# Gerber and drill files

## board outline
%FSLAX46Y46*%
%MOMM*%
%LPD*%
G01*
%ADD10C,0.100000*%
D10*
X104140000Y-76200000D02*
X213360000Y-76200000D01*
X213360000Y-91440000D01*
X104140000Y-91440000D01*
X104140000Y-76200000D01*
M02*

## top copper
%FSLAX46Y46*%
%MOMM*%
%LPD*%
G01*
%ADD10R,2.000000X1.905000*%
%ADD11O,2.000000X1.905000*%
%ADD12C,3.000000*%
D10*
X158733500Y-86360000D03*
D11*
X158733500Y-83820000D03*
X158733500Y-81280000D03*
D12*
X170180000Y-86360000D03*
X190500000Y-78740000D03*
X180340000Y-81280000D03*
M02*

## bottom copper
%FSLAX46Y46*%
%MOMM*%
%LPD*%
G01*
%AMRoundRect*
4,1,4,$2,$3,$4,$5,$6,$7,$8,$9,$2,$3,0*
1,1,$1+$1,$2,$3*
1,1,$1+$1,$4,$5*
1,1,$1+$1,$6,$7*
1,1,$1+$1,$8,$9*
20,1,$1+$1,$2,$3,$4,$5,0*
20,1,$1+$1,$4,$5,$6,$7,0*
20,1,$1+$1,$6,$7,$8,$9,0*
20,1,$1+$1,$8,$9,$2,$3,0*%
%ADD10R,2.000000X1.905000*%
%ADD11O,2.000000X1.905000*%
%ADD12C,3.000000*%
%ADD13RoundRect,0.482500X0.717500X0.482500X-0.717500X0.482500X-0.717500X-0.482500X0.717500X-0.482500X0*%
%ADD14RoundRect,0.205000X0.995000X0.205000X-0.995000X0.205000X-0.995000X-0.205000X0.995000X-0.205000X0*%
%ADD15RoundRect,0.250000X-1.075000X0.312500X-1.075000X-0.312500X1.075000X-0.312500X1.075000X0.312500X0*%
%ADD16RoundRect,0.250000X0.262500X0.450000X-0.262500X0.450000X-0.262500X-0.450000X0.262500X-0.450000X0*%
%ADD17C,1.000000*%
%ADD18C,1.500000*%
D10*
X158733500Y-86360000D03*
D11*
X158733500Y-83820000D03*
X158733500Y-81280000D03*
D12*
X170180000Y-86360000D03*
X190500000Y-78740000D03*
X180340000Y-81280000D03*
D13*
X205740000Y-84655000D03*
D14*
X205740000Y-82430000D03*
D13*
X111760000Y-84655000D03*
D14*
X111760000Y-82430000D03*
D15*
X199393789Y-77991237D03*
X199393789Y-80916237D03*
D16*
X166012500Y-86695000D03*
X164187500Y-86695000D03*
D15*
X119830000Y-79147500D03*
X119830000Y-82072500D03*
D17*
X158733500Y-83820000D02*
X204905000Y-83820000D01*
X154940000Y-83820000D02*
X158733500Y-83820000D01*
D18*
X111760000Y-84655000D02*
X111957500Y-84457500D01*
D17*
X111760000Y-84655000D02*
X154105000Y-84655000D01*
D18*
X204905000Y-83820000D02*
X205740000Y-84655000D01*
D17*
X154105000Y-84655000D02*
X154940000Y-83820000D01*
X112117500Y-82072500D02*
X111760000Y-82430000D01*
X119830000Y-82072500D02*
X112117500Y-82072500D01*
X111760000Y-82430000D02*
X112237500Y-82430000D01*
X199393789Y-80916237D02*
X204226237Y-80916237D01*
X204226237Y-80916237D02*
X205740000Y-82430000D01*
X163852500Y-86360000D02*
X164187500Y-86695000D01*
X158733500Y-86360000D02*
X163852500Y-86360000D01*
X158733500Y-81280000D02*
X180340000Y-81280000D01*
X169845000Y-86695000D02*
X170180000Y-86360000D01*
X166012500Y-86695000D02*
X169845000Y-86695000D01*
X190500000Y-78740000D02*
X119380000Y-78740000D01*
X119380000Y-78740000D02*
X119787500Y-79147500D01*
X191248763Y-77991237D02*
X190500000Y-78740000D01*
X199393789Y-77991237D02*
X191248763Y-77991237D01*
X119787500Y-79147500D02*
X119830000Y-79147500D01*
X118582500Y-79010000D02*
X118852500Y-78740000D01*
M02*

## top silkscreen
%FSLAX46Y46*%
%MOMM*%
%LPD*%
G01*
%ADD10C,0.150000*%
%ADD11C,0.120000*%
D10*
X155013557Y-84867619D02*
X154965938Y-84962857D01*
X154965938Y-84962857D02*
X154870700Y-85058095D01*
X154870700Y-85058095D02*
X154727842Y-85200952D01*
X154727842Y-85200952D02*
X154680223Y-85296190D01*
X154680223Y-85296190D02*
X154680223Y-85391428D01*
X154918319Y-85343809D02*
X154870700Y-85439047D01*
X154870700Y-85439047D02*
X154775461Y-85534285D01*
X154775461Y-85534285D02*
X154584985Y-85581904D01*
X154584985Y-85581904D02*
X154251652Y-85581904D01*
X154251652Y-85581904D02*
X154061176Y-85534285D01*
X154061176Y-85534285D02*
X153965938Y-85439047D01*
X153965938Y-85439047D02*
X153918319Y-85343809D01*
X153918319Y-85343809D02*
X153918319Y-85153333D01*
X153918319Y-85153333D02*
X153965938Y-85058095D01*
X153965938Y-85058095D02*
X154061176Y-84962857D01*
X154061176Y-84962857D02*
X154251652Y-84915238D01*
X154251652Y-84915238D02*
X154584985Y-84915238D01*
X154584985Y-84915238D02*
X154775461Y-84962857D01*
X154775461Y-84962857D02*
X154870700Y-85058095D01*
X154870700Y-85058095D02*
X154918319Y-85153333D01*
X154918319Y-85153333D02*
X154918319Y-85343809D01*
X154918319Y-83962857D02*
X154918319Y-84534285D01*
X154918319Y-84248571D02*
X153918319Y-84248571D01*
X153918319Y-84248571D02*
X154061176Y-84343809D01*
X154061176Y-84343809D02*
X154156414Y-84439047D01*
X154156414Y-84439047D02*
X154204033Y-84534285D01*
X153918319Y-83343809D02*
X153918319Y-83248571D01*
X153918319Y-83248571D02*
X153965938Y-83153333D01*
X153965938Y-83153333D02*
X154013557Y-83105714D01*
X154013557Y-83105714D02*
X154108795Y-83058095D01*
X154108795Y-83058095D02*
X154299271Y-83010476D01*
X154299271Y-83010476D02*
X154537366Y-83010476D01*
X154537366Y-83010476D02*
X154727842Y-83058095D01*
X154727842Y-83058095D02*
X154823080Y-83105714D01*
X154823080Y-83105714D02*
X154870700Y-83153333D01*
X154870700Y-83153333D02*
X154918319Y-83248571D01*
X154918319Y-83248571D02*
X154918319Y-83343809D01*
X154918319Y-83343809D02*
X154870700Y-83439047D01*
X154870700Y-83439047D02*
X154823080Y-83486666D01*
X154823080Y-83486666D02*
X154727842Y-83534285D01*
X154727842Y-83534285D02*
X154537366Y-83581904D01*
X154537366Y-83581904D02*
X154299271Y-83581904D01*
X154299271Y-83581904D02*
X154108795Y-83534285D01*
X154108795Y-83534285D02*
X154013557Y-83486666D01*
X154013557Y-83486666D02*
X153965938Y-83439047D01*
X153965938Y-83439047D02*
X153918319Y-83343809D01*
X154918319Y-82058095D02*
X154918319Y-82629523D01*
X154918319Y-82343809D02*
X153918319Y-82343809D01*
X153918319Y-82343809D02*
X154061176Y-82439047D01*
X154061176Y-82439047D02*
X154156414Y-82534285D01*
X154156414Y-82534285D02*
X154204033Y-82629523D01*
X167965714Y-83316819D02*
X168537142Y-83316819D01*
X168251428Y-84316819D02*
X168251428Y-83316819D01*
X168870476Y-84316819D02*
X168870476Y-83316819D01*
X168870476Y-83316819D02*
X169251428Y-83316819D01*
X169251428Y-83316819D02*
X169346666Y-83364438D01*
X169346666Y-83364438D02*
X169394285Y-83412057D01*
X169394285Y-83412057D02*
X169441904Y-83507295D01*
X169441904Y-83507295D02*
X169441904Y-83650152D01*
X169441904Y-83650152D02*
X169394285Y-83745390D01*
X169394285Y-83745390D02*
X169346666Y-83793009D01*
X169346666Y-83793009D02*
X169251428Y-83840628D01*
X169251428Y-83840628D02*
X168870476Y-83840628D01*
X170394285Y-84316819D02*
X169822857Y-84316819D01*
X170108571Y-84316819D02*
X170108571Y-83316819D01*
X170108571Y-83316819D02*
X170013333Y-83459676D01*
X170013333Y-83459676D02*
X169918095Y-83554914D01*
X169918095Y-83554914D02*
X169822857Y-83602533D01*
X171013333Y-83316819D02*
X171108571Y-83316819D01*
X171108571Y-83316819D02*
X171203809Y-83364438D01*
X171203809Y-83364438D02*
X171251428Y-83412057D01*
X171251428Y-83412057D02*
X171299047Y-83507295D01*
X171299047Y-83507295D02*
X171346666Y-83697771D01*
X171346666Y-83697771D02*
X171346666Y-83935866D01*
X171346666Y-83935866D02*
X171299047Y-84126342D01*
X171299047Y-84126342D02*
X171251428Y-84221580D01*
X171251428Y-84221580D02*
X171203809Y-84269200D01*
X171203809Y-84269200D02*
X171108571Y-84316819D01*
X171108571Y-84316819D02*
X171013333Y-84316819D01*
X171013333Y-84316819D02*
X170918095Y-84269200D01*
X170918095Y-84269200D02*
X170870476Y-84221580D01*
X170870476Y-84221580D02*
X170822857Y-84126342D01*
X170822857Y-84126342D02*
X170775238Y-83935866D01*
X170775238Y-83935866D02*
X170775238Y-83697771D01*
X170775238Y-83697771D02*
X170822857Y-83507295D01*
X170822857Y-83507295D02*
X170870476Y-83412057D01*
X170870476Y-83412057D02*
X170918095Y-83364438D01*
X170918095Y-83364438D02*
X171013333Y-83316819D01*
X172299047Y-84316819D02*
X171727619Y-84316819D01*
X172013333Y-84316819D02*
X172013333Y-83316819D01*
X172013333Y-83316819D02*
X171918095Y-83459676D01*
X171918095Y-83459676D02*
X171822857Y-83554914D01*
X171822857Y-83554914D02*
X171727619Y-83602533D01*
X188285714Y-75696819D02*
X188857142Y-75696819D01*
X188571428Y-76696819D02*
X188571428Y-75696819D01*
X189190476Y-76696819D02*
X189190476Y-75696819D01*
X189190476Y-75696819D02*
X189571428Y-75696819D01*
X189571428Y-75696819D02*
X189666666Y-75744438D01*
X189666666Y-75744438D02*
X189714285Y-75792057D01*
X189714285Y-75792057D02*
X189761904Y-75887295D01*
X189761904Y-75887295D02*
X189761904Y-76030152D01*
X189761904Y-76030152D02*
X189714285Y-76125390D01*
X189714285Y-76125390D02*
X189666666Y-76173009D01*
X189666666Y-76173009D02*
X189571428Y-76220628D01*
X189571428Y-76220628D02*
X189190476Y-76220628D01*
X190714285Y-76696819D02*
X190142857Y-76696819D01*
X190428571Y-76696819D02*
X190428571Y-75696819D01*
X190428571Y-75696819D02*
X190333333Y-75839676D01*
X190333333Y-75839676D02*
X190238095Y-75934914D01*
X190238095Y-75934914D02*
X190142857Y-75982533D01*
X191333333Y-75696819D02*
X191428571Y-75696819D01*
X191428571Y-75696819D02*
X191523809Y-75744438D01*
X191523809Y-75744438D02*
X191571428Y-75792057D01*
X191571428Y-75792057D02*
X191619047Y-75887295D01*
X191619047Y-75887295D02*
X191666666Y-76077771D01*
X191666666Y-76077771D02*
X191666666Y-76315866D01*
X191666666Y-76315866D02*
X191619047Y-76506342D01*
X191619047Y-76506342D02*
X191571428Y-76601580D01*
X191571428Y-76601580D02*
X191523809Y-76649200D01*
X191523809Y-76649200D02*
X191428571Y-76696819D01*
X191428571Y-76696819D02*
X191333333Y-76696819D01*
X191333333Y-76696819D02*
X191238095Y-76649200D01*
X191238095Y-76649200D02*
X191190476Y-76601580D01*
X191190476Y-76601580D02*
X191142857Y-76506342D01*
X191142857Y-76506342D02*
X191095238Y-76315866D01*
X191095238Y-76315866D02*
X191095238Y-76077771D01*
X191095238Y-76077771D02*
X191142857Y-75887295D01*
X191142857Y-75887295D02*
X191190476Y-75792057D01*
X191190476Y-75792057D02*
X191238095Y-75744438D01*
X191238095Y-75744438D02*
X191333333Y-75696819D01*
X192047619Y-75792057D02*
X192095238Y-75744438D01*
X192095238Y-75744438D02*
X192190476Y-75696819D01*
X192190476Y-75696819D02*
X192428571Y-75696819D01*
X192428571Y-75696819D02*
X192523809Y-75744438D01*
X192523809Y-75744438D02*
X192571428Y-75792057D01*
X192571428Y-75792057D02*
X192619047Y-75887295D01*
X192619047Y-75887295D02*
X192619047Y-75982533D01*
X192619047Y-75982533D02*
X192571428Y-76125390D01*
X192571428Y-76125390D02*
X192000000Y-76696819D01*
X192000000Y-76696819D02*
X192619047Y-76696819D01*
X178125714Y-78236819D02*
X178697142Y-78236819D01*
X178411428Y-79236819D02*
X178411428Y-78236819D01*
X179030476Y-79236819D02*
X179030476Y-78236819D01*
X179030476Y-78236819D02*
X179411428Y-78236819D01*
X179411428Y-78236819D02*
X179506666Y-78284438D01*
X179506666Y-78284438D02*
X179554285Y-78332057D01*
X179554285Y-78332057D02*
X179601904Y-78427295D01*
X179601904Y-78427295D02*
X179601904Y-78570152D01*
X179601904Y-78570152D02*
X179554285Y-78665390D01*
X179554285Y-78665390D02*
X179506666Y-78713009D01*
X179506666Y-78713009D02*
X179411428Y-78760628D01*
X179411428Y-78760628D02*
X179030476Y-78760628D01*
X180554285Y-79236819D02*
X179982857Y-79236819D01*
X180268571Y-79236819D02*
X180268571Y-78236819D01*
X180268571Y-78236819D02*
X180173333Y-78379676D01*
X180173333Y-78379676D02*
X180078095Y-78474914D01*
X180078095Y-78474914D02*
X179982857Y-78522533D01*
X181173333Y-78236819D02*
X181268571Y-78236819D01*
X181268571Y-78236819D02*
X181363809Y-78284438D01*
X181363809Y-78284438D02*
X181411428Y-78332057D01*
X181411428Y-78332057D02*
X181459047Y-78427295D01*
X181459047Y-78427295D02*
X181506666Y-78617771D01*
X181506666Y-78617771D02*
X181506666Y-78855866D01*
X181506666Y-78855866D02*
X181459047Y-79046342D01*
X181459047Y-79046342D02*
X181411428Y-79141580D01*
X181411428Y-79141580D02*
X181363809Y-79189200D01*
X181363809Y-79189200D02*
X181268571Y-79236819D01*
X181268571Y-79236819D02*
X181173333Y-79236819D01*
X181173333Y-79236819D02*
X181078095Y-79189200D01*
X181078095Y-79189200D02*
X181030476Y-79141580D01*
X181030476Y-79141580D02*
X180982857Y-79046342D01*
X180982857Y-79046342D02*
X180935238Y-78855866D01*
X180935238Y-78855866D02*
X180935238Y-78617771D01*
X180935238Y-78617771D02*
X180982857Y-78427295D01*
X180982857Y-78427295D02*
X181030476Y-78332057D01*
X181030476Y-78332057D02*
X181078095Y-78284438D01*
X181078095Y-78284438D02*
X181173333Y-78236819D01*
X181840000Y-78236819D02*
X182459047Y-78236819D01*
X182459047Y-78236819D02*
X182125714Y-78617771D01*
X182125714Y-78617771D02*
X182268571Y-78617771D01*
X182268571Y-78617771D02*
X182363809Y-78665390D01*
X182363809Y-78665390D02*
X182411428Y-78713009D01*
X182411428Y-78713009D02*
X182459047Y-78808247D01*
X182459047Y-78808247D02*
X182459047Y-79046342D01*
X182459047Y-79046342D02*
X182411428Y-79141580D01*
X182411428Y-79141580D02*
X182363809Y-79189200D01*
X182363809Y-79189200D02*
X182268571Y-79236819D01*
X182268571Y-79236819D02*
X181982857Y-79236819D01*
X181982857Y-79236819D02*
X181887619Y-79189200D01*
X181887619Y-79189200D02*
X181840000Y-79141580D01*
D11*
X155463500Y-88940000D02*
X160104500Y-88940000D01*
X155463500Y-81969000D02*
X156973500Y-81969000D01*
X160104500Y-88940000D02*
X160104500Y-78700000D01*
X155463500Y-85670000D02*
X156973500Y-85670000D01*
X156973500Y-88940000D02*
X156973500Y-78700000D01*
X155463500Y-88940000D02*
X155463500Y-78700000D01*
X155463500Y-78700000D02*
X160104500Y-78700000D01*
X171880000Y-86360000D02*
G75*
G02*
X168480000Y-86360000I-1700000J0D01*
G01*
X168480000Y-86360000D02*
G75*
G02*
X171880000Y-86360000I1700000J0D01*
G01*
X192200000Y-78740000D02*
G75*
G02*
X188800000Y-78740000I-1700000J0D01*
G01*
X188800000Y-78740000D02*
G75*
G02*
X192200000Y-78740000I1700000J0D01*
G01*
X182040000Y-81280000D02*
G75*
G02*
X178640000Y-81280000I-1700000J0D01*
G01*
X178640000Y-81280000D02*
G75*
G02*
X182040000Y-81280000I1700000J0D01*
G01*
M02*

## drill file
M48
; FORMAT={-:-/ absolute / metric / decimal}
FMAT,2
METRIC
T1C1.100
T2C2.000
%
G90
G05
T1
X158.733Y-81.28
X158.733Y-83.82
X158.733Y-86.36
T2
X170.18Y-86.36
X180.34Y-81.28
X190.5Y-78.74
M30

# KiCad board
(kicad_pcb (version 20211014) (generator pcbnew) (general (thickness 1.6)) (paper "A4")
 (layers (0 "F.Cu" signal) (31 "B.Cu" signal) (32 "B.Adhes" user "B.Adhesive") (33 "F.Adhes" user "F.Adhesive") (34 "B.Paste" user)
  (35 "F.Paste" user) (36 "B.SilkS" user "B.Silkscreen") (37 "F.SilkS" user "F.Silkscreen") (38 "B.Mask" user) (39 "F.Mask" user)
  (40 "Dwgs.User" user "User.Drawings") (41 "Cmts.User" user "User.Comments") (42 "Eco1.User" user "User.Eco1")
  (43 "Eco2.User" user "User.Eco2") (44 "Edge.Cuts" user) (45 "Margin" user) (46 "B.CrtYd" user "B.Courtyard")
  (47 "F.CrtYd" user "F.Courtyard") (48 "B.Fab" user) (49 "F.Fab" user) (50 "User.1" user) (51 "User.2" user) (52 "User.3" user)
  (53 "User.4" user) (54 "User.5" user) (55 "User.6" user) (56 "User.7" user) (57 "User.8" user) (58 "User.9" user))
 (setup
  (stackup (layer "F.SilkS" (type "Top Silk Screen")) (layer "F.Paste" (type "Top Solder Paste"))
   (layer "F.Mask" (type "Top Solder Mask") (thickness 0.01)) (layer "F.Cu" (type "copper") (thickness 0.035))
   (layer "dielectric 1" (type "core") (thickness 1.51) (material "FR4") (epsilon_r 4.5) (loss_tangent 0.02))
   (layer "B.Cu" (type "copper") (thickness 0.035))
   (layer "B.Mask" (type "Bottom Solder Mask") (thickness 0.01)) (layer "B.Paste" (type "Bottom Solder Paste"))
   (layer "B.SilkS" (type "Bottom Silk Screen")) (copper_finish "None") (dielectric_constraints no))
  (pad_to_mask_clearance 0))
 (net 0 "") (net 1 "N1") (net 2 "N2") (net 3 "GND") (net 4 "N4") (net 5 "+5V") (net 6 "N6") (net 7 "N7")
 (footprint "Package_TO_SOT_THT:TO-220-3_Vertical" (layer "F.Cu") (at 158.7335 86.36 90)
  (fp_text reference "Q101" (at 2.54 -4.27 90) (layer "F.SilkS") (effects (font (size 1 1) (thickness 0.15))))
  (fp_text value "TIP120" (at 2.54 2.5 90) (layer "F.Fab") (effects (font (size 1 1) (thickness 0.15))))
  (fp_line (start -2.58 -3.27) (end -2.58 1.371) (layer "F.SilkS") (width 0.12))
  (fp_line (start 4.391 -3.27) (end 4.391 -1.76) (layer "F.SilkS") (width 0.12))
  (fp_line (start -2.58 1.371) (end 7.66 1.371) (layer "F.SilkS") (width 0.12))
  (fp_line (start 0.69 -3.27) (end 0.69 -1.76) (layer "F.SilkS") (width 0.12))
  (fp_line (start -2.58 -1.76) (end 7.66 -1.76) (layer "F.SilkS") (width 0.12))
  (fp_line (start -2.58 -3.27) (end 7.66 -3.27) (layer "F.SilkS") (width 0.12))
  (fp_line (start 7.66 -3.27) (end 7.66 1.371) (layer "F.SilkS") (width 0.12))
  (pad "1" thru_hole rect (at 0 0 90) (size 1.905 2) (drill 1.1) (layers *.Cu *.Mask) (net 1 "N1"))
  (pad "2" thru_hole oval (at 2.54 0 90) (size 1.905 2) (drill 1.1) (layers *.Cu *.Mask) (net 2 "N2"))
  (pad "3" thru_hole oval (at 5.08 0 90) (size 1.905 2) (drill 1.1) (layers *.Cu *.Mask) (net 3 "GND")))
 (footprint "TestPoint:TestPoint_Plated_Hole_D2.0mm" (layer "F.Cu") (at 170.18 86.36)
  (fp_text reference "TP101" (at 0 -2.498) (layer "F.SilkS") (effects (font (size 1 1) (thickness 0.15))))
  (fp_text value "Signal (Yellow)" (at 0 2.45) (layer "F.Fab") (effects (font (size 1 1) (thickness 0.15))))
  (fp_circle (center 0 0) (end 0 -1.7) (layer "F.SilkS") (width 0.12) (fill none))
  (pad "1" thru_hole circle (at 0 0) (size 3 3) (drill 2) (layers *.Cu *.Mask) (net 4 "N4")))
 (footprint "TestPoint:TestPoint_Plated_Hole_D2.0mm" (layer "F.Cu") (at 190.5 78.74)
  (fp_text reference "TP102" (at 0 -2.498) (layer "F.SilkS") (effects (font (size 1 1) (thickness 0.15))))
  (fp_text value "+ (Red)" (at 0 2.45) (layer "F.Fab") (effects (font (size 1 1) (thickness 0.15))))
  (fp_circle (center 0 0) (end 0 -1.7) (layer "F.SilkS") (width 0.12) (fill none))
  (pad "1" thru_hole circle (at 0 0) (size 3 3) (drill 2) (layers *.Cu *.Mask) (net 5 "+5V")))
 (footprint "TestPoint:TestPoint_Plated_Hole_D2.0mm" (layer "F.Cu") (at 180.34 81.28)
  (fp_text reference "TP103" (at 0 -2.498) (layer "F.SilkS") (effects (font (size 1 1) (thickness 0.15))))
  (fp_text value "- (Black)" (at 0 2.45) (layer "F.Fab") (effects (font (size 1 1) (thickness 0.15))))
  (fp_circle (center 0 0) (end 0 -1.7) (layer "F.SilkS") (width 0.12) (fill none))
  (pad "1" thru_hole circle (at 0 0) (size 3 3) (drill 2) (layers *.Cu *.Mask) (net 3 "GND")))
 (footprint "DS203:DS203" (layer "B.Cu") (at 205.74 83.82 180)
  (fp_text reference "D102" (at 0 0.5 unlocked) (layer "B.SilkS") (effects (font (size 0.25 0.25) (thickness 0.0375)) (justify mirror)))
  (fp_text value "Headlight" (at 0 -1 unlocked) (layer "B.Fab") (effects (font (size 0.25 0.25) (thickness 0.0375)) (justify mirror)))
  (pad "1" smd roundrect (at 0 -0.835 180) (size 2.4 1.93) (layers "B.Cu" "B.Paste" "B.Mask") (roundrect_rratio 0.25) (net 2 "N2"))
  (pad "2" smd roundrect (at 0 1.39 180) (size 2.4 0.82) (layers "B.Cu" "B.Paste" "B.Mask") (roundrect_rratio 0.25) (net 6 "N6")))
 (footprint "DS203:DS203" (layer "B.Cu") (at 111.76 83.82 180)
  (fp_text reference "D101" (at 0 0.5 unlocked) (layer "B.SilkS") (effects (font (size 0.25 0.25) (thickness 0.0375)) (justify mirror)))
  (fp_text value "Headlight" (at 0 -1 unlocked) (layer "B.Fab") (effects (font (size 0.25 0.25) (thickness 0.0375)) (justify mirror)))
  (pad "1" smd roundrect (at 0 -0.835 180) (size 2.4 1.93) (layers "B.Cu" "B.Paste" "B.Mask") (roundrect_rratio 0.25) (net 2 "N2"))
  (pad "2" smd roundrect (at 0 1.39 180) (size 2.4 0.82) (layers "B.Cu" "B.Paste" "B.Mask") (roundrect_rratio 0.25) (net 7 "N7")))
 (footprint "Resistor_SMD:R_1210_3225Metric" (layer "B.Cu") (at 199.393789 79.453737 -90)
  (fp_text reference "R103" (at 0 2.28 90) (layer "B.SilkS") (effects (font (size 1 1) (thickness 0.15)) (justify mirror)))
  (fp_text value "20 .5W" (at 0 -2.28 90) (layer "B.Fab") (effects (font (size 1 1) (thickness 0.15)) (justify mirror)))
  (pad "1" smd roundrect (at -1.4625 0 270) (size 1.125 2.65) (layers "B.Cu" "B.Paste" "B.Mask") (roundrect_rratio 0.2222222222)
   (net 5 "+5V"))
  (pad "2" smd roundrect (at 1.4625 0 270) (size 1.125 2.65) (layers "B.Cu" "B.Paste" "B.Mask") (roundrect_rratio 0.2222222222) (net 6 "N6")))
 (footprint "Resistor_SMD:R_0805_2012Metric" (layer "B.Cu") (at 165.1 86.695 180)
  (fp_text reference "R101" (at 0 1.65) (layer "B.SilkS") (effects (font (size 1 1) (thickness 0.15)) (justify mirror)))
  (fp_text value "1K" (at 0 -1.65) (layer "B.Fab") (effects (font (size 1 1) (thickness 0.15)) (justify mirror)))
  (pad "1" smd roundrect (at -0.9125 0 180) (size 1.025 1.4) (layers "B.Cu" "B.Paste" "B.Mask") (roundrect_rratio 0.243902439) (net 4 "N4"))
  (pad "2" smd roundrect (at 0.9125 0 180) (size 1.025 1.4) (layers "B.Cu" "B.Paste" "B.Mask") (roundrect_rratio 0.243902439) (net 1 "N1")))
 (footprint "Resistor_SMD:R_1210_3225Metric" (layer "B.Cu") (at 119.83 80.61 -90)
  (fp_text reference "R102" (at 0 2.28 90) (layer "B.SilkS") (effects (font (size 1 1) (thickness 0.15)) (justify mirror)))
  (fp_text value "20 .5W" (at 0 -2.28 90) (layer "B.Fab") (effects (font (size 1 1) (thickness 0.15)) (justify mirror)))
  (pad "1" smd roundrect (at -1.4625 0 270) (size 1.125 2.65) (layers "B.Cu" "B.Paste" "B.Mask") (roundrect_rratio 0.2222222222)
   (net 5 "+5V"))
  (pad "2" smd roundrect (at 1.4625 0 270) (size 1.125 2.65) (layers "B.Cu" "B.Paste" "B.Mask") (roundrect_rratio 0.2222222222) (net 7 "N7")))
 (gr_rect (start 104.14 76.2) (end 213.36 91.44) (layer "Edge.Cuts") (width 0.1) (fill none))
 (segment (start 158.7335 83.82) (end 204.905 83.82) (width 1) (layer "B.Cu") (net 2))
 (segment (start 154.94 83.82) (end 158.7335 83.82) (width 1) (layer "B.Cu") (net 2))
 (segment (start 111.76 84.655) (end 111.9575 84.4575) (width 1.5) (layer "B.Cu") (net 2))
 (segment (start 111.76 84.655) (end 154.105 84.655) (width 1) (layer "B.Cu") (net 2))
 (segment (start 204.905 83.82) (end 205.74 84.655) (width 1.5) (layer "B.Cu") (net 2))
 (segment (start 154.105 84.655) (end 154.94 83.82) (width 1) (layer "B.Cu") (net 2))
 (segment (start 112.1175 82.0725) (end 111.76 82.43) (width 1) (layer "B.Cu") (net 7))
 (segment (start 119.83 82.0725) (end 112.1175 82.0725) (width 1) (layer "B.Cu") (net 7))
 (segment (start 111.76 82.43) (end 112.2375 82.43) (width 1) (layer "B.Cu") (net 7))
 (segment (start 199.393789 80.916237) (end 204.226237 80.916237) (width 1) (layer "B.Cu") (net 6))
 (segment (start 204.226237 80.916237) (end 205.74 82.43) (width 1) (layer "B.Cu") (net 6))
 (segment (start 163.8525 86.36) (end 164.1875 86.695) (width 1) (layer "B.Cu") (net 1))
 (segment (start 158.7335 86.36) (end 163.8525 86.36) (width 1) (layer "B.Cu") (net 1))
 (segment (start 158.7335 81.28) (end 180.34 81.28) (width 1) (layer "B.Cu") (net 3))
 (segment (start 169.845 86.695) (end 170.18 86.36) (width 1) (layer "B.Cu") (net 4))
 (segment (start 166.0125 86.695) (end 169.845 86.695) (width 1) (layer "B.Cu") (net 4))
 (segment (start 190.5 78.74) (end 119.38 78.74) (width 1) (layer "B.Cu") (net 5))
 (segment (start 119.38 78.74) (end 119.7875 79.1475) (width 1) (layer "B.Cu") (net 5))
 (segment (start 191.248763 77.991237) (end 190.5 78.74) (width 1) (layer "B.Cu") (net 5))
 (segment (start 199.393789 77.991237) (end 191.248763 77.991237) (width 1) (layer "B.Cu") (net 5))
 (segment (start 119.7875 79.1475) (end 119.83 79.1475) (width 1) (layer "B.Cu") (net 5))
 (segment (start 118.5825 79.01) (end 118.8525 78.74) (width 1) (layer "B.Cu") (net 5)))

